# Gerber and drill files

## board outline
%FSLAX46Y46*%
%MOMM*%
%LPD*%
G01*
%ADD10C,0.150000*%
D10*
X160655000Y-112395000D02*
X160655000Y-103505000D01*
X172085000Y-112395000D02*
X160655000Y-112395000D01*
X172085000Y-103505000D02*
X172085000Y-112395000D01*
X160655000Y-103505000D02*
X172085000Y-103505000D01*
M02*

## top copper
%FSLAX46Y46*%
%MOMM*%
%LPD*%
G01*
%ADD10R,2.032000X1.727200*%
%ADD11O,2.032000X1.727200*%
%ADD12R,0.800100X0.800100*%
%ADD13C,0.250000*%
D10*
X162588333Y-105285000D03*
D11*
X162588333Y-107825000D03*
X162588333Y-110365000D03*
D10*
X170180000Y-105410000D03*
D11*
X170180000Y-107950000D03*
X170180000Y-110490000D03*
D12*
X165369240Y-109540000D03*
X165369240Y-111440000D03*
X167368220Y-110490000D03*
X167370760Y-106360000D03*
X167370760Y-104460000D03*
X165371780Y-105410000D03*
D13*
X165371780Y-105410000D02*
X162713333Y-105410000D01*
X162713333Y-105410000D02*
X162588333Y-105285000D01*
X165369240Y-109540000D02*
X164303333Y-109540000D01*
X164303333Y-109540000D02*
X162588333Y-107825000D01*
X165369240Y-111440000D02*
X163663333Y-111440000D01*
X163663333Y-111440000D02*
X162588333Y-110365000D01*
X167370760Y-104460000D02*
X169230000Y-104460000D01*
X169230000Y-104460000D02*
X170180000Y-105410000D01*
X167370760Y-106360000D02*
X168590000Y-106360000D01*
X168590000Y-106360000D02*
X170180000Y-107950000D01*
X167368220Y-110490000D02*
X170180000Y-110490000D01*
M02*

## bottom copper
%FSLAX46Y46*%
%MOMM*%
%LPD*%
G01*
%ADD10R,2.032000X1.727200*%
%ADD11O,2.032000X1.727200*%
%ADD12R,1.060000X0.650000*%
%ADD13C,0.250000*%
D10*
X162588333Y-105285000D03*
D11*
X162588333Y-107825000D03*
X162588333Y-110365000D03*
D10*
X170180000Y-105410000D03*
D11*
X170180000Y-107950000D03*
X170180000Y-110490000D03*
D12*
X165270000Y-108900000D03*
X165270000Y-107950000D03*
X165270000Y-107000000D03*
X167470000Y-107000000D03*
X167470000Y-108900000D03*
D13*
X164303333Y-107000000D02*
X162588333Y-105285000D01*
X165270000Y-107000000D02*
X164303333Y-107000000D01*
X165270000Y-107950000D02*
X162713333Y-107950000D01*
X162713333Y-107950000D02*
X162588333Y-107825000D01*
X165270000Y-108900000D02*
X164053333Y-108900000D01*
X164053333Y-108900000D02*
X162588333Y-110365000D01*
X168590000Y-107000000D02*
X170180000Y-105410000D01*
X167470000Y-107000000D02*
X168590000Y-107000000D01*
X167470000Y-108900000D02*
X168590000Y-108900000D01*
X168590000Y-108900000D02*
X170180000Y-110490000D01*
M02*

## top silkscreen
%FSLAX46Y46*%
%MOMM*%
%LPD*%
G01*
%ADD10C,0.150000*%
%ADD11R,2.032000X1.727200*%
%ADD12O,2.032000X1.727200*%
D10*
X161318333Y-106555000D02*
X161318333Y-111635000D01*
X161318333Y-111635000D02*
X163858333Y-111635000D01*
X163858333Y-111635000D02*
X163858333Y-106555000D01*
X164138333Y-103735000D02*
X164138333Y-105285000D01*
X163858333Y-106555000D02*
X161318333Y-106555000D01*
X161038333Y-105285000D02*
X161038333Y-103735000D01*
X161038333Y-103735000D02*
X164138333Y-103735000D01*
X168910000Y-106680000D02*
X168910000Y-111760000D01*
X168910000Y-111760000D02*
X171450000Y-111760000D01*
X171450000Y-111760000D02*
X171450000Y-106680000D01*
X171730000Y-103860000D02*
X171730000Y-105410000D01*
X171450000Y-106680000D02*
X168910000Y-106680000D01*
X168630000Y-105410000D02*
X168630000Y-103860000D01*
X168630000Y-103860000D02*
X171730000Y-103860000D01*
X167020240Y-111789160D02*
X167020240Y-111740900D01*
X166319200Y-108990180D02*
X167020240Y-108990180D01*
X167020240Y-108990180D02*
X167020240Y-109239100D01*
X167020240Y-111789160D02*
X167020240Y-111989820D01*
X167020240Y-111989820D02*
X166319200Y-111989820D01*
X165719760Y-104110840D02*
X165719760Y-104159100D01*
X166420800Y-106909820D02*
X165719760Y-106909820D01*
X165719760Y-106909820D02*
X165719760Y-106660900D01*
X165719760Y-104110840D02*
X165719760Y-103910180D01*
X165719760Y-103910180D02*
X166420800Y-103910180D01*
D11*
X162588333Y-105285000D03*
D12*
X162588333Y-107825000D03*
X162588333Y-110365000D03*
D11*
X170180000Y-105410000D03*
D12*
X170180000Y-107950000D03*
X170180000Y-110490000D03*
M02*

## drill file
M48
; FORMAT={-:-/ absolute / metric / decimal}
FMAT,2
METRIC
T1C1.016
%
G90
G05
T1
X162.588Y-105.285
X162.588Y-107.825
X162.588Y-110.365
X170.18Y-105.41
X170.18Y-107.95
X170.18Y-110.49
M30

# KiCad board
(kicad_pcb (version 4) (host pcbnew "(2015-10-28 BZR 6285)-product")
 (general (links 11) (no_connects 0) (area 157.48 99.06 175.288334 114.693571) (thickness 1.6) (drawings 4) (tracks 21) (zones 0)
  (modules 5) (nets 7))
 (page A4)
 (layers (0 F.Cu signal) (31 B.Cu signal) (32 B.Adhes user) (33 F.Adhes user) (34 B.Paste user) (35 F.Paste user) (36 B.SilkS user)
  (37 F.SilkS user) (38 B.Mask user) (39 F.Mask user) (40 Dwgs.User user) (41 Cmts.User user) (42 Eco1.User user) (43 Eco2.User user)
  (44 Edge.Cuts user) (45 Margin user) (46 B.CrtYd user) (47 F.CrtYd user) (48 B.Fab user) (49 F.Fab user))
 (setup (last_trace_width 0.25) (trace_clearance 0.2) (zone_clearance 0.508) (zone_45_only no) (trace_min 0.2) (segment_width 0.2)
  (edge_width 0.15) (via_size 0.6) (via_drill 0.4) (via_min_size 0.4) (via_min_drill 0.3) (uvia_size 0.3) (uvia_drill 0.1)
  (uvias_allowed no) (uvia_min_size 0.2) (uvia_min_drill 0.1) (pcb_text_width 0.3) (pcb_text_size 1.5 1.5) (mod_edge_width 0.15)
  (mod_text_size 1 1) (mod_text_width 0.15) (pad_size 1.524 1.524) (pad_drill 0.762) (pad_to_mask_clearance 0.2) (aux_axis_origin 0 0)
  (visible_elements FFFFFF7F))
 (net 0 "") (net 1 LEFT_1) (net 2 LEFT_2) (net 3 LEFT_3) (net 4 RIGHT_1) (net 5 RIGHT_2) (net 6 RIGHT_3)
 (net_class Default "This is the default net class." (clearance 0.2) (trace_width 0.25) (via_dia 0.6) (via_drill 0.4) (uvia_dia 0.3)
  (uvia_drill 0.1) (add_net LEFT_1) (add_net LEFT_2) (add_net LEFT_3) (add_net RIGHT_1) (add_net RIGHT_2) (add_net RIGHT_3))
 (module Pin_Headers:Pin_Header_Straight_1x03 (layer F.Cu) (at 162.588333 105.285)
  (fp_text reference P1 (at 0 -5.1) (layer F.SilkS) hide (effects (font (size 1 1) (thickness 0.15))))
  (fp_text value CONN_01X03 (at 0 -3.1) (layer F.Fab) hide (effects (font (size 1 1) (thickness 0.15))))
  (fp_line (start -1.27 1.27) (end -1.27 6.35) (layer F.SilkS) (width 0.15))
  (fp_line (start -1.27 6.35) (end 1.27 6.35) (layer F.SilkS) (width 0.15))
  (fp_line (start 1.27 6.35) (end 1.27 1.27) (layer F.SilkS) (width 0.15))
  (fp_line (start 1.55 -1.55) (end 1.55 0) (layer F.SilkS) (width 0.15))
  (fp_line (start 1.27 1.27) (end -1.27 1.27) (layer F.SilkS) (width 0.15))
  (fp_line (start -1.55 0) (end -1.55 -1.55) (layer F.SilkS) (width 0.15))
  (fp_line (start -1.55 -1.55) (end 1.55 -1.55) (layer F.SilkS) (width 0.15))
  (pad 1 thru_hole rect (at 0 0) (size 2.032 1.7272) (drill 1.016) (layers *.Cu *.Mask F.SilkS) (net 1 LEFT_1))
  (pad 2 thru_hole oval (at 0 2.54) (size 2.032 1.7272) (drill 1.016) (layers *.Cu *.Mask F.SilkS) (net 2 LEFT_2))
  (pad 3 thru_hole oval (at 0 5.08) (size 2.032 1.7272) (drill 1.016) (layers *.Cu *.Mask F.SilkS) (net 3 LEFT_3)))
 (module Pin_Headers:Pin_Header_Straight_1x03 (layer F.Cu) (at 170.18 105.41)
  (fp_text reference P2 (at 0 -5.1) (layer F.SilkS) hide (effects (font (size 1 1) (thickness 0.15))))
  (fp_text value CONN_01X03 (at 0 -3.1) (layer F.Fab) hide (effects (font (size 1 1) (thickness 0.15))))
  (fp_line (start -1.27 1.27) (end -1.27 6.35) (layer F.SilkS) (width 0.15))
  (fp_line (start -1.27 6.35) (end 1.27 6.35) (layer F.SilkS) (width 0.15))
  (fp_line (start 1.27 6.35) (end 1.27 1.27) (layer F.SilkS) (width 0.15))
  (fp_line (start 1.55 -1.55) (end 1.55 0) (layer F.SilkS) (width 0.15))
  (fp_line (start 1.27 1.27) (end -1.27 1.27) (layer F.SilkS) (width 0.15))
  (fp_line (start -1.55 0) (end -1.55 -1.55) (layer F.SilkS) (width 0.15))
  (fp_line (start -1.55 -1.55) (end 1.55 -1.55) (layer F.SilkS) (width 0.15))
  (pad 1 thru_hole rect (at 0 0) (size 2.032 1.7272) (drill 1.016) (layers *.Cu *.Mask F.SilkS) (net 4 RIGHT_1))
  (pad 2 thru_hole oval (at 0 2.54) (size 2.032 1.7272) (drill 1.016) (layers *.Cu *.Mask F.SilkS) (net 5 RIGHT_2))
  (pad 3 thru_hole oval (at 0 5.08) (size 2.032 1.7272) (drill 1.016) (layers *.Cu *.Mask F.SilkS) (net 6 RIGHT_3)))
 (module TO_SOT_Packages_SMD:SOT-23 (layer F.Cu) (at 166.37 110.49 270)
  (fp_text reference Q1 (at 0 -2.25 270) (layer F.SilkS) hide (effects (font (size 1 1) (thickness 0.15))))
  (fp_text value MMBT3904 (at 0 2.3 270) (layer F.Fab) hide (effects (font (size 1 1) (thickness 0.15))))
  (fp_line (start 1.29916 -0.65024) (end 1.2509 -0.65024) (layer F.SilkS) (width 0.15))
  (fp_line (start -1.49982 0.0508) (end -1.49982 -0.65024) (layer F.SilkS) (width 0.15))
  (fp_line (start -1.49982 -0.65024) (end -1.2509 -0.65024) (layer F.SilkS) (width 0.15))
  (fp_line (start 1.29916 -0.65024) (end 1.49982 -0.65024) (layer F.SilkS) (width 0.15))
  (fp_line (start 1.49982 -0.65024) (end 1.49982 0.0508) (layer F.SilkS) (width 0.15))
  (pad 1 smd rect (at -0.95 1.00076 270) (size 0.8001 0.8001) (layers F.Cu F.Paste F.Mask) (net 2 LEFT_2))
  (pad 2 smd rect (at 0.95 1.00076 270) (size 0.8001 0.8001) (layers F.Cu F.Paste F.Mask) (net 3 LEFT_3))
  (pad 3 smd rect (at 0 -0.99822 270) (size 0.8001 0.8001) (layers F.Cu F.Paste F.Mask) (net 6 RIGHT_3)))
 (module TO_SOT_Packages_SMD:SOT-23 (layer F.Cu) (at 166.37 105.41 90)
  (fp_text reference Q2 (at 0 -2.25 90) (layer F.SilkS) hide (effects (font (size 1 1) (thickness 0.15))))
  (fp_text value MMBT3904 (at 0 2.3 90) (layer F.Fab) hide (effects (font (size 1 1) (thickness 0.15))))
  (fp_line (start 1.29916 -0.65024) (end 1.2509 -0.65024) (layer F.SilkS) (width 0.15))
  (fp_line (start -1.49982 0.0508) (end -1.49982 -0.65024) (layer F.SilkS) (width 0.15))
  (fp_line (start -1.49982 -0.65024) (end -1.2509 -0.65024) (layer F.SilkS) (width 0.15))
  (fp_line (start 1.29916 -0.65024) (end 1.49982 -0.65024) (layer F.SilkS) (width 0.15))
  (fp_line (start 1.49982 -0.65024) (end 1.49982 0.0508) (layer F.SilkS) (width 0.15))
  (pad 1 smd rect (at -0.95 1.00076 90) (size 0.8001 0.8001) (layers F.Cu F.Paste F.Mask) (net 5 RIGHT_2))
  (pad 2 smd rect (at 0.95 1.00076 90) (size 0.8001 0.8001) (layers F.Cu F.Paste F.Mask) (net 4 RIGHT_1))
  (pad 3 smd rect (at 0 -0.99822 90) (size 0.8001 0.8001) (layers F.Cu F.Paste F.Mask) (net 1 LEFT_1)))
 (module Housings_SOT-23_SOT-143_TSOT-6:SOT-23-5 (layer B.Cu) (at 166.37 107.95) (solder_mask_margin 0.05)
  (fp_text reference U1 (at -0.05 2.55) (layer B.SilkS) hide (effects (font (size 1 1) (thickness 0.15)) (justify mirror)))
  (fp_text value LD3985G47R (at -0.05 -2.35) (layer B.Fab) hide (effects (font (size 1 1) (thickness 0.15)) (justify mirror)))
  (pad 1 smd rect (at -1.1 0.95) (size 1.06 0.65) (layers B.Cu B.Paste B.Mask) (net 3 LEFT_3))
  (pad 2 smd rect (at -1.1 0) (size 1.06 0.65) (layers B.Cu B.Paste B.Mask) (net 2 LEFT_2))
  (pad 3 smd rect (at -1.1 -0.95) (size 1.06 0.65) (layers B.Cu B.Paste B.Mask) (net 1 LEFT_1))
  (pad 4 smd rect (at 1.1 -0.95) (size 1.06 0.65) (layers B.Cu B.Paste B.Mask) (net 4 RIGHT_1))
  (pad 5 smd rect (at 1.1 0.95) (size 1.06 0.65) (layers B.Cu B.Paste B.Mask) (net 6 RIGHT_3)))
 (gr_line (start 160.655 112.395) (end 160.655 103.505) (angle 90) (layer Edge.Cuts) (width 0.15))
 (gr_line (start 172.085 112.395) (end 160.655 112.395) (angle 90) (layer Edge.Cuts) (width 0.15))
 (gr_line (start 172.085 103.505) (end 172.085 112.395) (angle 90) (layer Edge.Cuts) (width 0.15))
 (gr_line (start 160.655 103.505) (end 172.085 103.505) (angle 90) (layer Edge.Cuts) (width 0.15))
 (segment (start 164.303333 107) (end 162.588333 105.285) (width 0.25) (layer B.Cu) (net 1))
 (segment (start 165.37178 105.41) (end 162.713333 105.41) (width 0.25) (layer F.Cu) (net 1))
 (segment (start 162.713333 105.41) (end 162.588333 105.285) (width 0.25) (layer F.Cu) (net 1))
 (segment (start 165.27 107) (end 164.303333 107) (width 0.25) (layer B.Cu) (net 1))
 (segment (start 165.27 107.95) (end 162.713333 107.95) (width 0.25) (layer B.Cu) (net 2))
 (segment (start 162.713333 107.95) (end 162.588333 107.825) (width 0.25) (layer B.Cu) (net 2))
 (segment (start 165.36924 109.54) (end 164.303333 109.54) (width 0.25) (layer F.Cu) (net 2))
 (segment (start 164.303333 109.54) (end 162.588333 107.825) (width 0.25) (layer F.Cu) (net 2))
 (segment (start 165.27 108.9) (end 164.053333 108.9) (width 0.25) (layer B.Cu) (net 3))
 (segment (start 164.053333 108.9) (end 162.588333 110.365) (width 0.25) (layer B.Cu) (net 3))
 (segment (start 165.36924 111.44) (end 163.663333 111.44) (width 0.25) (layer F.Cu) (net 3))
 (segment (start 163.663333 111.44) (end 162.588333 110.365) (width 0.25) (layer F.Cu) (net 3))
 (segment (start 168.59 107) (end 170.18 105.41) (width 0.25) (layer B.Cu) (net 4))
 (segment (start 167.37076 104.46) (end 169.23 104.46) (width 0.25) (layer F.Cu) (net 4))
 (segment (start 169.23 104.46) (end 170.18 105.41) (width 0.25) (layer F.Cu) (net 4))
 (segment (start 167.47 107) (end 168.59 107) (width 0.25) (layer B.Cu) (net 4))
 (segment (start 167.37076 106.36) (end 168.59 106.36) (width 0.25) (layer F.Cu) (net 5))
 (segment (start 168.59 106.36) (end 170.18 107.95) (width 0.25) (layer F.Cu) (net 5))
 (segment (start 167.47 108.9) (end 168.59 108.9) (width 0.25) (layer B.Cu) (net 6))
 (segment (start 168.59 108.9) (end 170.18 110.49) (width 0.25) (layer B.Cu) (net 6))
 (segment (start 167.36822 110.49) (end 170.18 110.49) (width 0.25) (layer F.Cu) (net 6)))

